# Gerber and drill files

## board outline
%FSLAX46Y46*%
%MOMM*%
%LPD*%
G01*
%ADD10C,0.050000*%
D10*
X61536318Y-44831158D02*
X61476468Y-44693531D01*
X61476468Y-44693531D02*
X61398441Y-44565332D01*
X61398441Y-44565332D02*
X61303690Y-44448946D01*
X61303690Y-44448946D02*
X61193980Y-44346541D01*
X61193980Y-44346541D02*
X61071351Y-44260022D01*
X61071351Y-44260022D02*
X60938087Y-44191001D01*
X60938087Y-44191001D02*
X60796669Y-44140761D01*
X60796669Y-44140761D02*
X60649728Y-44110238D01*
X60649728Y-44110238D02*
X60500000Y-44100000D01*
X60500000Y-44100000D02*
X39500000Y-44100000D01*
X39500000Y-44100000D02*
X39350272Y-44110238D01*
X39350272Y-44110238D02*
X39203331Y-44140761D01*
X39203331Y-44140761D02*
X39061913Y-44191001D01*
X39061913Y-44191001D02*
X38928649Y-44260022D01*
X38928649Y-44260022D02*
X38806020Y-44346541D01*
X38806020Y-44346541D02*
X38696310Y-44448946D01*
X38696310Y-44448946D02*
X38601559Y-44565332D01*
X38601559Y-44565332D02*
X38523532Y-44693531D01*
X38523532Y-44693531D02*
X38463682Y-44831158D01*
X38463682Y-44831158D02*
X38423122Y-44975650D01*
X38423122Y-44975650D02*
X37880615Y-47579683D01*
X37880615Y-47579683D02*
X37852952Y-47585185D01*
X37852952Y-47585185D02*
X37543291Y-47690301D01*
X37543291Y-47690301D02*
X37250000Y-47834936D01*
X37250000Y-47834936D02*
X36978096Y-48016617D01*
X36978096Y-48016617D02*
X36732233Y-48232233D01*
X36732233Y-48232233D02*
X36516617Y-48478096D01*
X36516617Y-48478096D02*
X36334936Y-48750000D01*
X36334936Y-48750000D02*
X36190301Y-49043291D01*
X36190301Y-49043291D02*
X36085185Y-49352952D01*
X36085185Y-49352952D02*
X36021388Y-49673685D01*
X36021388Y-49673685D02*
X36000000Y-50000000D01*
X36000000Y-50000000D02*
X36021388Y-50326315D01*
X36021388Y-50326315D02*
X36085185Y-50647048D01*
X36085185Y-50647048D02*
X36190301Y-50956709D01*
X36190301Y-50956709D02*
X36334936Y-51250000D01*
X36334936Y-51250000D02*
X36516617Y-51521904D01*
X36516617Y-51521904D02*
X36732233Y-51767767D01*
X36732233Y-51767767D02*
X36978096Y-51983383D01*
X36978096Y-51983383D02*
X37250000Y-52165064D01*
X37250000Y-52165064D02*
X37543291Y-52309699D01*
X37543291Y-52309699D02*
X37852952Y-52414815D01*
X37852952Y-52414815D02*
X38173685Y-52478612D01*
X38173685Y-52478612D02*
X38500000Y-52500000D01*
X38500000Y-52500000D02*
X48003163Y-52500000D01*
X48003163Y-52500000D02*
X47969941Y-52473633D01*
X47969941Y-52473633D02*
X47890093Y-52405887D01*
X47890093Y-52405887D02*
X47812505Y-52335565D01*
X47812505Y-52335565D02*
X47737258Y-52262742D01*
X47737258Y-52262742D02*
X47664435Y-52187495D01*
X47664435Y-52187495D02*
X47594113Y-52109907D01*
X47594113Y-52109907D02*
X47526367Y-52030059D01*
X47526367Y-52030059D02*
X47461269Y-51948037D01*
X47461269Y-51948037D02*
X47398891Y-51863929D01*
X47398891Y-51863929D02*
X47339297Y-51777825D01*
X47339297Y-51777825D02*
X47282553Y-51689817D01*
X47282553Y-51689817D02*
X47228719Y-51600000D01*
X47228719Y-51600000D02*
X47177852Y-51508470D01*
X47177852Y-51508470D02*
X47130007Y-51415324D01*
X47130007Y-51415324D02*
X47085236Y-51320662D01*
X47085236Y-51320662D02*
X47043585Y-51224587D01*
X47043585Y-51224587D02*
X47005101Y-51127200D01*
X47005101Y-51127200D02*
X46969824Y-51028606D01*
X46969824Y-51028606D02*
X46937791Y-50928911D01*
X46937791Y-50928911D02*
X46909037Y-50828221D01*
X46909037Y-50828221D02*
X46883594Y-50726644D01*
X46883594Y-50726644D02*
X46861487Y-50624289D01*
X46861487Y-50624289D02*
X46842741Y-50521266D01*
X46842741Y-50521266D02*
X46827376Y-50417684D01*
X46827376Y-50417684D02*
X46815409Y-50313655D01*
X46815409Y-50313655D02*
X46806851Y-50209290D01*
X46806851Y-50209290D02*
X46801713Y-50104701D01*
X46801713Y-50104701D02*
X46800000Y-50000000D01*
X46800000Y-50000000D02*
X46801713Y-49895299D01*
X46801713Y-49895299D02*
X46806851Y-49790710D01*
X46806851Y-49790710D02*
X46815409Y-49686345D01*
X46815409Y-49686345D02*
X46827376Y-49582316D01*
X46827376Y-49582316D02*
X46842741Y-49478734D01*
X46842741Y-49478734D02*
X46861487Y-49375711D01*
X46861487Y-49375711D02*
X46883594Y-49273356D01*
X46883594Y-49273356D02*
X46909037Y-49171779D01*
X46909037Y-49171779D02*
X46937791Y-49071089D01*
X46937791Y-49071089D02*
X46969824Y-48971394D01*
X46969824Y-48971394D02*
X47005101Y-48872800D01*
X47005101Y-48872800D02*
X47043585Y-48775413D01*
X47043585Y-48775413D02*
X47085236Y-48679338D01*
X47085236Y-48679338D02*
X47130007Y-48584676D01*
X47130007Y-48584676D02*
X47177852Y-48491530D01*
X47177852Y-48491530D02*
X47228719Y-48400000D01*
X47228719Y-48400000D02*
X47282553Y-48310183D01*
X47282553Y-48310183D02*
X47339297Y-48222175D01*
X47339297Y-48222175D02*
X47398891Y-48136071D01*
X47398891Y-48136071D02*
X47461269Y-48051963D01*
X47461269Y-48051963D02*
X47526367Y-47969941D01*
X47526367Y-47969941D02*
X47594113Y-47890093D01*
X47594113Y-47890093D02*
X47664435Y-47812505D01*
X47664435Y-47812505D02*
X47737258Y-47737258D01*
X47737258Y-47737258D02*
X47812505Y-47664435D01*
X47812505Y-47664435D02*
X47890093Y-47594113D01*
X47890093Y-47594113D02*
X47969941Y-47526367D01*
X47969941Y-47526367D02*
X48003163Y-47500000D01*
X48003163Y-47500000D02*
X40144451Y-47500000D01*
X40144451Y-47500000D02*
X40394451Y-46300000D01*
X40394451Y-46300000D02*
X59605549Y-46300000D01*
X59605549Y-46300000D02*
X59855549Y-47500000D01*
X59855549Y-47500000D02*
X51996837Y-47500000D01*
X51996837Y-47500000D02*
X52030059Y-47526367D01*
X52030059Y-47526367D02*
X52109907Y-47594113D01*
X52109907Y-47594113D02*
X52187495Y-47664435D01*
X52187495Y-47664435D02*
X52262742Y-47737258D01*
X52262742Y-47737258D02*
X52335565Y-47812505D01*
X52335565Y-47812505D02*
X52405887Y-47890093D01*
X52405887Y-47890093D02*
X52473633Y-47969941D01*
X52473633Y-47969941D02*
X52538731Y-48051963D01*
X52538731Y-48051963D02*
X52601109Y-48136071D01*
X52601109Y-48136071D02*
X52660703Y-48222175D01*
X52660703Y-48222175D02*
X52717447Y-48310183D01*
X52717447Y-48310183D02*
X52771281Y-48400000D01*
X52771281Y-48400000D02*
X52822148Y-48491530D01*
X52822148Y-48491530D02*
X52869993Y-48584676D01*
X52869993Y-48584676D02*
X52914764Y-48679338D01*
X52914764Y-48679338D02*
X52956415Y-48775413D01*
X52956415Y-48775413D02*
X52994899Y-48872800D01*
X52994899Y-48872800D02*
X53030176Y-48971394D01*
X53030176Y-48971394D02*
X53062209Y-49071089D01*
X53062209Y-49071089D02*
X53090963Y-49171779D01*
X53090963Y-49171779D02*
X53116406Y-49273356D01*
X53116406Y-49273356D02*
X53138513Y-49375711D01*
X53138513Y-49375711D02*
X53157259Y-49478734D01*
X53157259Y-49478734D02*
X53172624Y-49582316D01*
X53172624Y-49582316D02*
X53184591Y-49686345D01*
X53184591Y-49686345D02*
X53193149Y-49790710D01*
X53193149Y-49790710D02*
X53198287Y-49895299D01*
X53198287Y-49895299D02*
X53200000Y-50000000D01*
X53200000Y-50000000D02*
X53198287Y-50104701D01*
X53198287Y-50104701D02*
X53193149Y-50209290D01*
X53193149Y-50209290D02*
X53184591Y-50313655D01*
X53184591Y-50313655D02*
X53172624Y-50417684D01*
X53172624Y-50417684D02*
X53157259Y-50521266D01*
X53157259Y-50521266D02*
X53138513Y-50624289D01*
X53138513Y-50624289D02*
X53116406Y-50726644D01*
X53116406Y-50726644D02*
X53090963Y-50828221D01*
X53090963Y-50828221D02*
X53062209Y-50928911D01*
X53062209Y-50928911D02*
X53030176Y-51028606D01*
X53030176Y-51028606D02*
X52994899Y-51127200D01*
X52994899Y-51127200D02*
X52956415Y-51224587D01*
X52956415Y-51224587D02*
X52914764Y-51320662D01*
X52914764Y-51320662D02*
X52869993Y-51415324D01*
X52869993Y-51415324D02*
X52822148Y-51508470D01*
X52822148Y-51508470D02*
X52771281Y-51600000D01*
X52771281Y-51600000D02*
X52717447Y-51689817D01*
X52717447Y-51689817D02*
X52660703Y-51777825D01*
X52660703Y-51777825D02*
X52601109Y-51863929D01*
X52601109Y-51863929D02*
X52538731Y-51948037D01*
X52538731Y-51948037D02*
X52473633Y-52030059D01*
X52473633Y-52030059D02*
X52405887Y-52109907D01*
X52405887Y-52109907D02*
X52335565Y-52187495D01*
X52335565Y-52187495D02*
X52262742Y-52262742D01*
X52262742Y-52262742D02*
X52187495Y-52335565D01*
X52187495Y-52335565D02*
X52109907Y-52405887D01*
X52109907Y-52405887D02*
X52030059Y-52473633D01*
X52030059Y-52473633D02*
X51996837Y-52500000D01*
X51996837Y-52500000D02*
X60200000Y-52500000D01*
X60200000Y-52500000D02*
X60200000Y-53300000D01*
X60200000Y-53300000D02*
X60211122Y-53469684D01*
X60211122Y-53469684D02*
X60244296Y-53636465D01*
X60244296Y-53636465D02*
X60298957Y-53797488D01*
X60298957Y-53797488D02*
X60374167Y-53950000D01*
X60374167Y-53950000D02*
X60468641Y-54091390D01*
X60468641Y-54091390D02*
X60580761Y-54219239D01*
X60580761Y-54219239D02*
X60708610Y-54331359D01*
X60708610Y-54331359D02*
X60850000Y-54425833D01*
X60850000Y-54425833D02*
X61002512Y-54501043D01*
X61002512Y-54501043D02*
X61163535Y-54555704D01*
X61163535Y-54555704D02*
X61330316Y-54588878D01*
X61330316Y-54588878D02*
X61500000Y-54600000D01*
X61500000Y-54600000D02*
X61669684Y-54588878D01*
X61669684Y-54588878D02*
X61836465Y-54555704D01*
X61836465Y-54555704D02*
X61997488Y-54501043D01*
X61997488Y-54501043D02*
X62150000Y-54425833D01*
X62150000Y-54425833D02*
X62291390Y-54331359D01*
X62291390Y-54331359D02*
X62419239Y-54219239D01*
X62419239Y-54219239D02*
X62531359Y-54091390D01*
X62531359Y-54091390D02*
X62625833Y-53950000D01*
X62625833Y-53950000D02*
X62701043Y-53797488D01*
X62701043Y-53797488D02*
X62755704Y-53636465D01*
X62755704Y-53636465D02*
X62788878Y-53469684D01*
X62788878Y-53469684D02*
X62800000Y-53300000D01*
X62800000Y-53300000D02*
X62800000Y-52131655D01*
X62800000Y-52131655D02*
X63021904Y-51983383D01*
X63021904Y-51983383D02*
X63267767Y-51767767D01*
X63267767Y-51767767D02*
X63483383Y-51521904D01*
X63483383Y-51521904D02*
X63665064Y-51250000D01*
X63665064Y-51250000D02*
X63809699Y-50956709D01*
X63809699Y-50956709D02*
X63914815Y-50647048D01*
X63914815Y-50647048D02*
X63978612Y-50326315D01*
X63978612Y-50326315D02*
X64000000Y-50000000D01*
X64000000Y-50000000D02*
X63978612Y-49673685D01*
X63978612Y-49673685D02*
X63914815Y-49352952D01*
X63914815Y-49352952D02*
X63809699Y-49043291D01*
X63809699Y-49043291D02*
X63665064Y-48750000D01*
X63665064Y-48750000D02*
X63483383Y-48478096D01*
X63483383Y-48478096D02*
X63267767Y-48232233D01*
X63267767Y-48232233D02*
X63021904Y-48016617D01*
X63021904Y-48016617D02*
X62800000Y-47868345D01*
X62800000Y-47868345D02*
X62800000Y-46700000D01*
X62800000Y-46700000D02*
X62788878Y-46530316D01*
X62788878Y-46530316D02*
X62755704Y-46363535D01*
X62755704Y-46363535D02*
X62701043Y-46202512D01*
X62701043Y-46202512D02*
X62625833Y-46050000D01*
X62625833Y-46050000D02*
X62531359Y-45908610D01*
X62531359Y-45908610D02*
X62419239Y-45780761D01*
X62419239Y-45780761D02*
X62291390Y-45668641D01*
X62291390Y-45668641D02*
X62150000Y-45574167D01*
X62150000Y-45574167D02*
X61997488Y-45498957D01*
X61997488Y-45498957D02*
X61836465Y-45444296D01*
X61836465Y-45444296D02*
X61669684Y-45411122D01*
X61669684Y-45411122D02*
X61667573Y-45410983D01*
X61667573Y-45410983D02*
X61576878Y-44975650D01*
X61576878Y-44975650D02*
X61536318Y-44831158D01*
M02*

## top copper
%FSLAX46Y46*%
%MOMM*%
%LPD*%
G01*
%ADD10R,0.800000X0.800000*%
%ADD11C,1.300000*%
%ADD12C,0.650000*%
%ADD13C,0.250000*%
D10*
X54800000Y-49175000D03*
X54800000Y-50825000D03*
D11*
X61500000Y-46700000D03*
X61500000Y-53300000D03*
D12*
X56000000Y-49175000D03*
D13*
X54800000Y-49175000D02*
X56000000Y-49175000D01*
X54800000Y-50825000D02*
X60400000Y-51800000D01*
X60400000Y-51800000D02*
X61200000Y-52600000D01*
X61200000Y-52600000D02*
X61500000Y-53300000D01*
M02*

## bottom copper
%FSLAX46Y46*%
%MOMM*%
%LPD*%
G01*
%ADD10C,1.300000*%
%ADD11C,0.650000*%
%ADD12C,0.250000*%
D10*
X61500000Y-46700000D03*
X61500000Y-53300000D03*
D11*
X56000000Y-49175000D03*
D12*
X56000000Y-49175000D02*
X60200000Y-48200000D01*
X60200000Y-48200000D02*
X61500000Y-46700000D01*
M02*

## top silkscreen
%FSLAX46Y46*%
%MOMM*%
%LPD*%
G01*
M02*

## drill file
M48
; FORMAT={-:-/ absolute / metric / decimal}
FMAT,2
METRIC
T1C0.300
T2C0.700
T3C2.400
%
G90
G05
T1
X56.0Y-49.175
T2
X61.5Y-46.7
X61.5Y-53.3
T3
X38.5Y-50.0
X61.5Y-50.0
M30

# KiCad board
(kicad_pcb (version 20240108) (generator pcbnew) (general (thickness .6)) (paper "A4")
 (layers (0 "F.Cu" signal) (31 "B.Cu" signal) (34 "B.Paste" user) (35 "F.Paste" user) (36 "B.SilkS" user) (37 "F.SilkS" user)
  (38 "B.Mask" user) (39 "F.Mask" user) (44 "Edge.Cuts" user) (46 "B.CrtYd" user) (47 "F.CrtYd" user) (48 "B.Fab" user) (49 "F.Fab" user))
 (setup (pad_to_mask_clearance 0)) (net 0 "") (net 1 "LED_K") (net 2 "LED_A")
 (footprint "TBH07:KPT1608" (layer "F.Cu") (at 54.8 50)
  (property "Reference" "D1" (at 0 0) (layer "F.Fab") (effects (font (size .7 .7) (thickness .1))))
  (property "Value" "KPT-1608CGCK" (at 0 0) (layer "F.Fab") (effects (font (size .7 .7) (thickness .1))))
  (pad "1" smd rect (at 0 -.825) (size .8 .8) (layers "F.Cu" "F.Paste" "F.Mask") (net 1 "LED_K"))
  (pad "2" smd rect (at 0 .825) (size .8 .8) (layers "F.Cu" "F.Paste" "F.Mask") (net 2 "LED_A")))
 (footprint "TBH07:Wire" (layer "F.Cu") (at 61.5 46.7)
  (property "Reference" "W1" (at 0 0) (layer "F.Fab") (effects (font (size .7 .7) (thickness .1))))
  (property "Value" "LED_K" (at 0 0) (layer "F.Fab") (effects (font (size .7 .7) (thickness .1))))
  (pad "1" thru_hole circle (at 0 0) (size 1.3 1.3) (drill .7) (layers "*.Cu" "*.Mask") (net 1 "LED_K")))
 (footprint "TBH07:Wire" (layer "F.Cu") (at 61.5 53.3)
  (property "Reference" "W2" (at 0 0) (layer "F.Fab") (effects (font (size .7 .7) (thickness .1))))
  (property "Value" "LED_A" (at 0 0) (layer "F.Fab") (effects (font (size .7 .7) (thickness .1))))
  (pad "1" thru_hole circle (at 0 0) (size 1.3 1.3) (drill .7) (layers "*.Cu" "*.Mask") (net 2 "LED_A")))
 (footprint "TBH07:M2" (layer "F.Cu") (at 38.5 50)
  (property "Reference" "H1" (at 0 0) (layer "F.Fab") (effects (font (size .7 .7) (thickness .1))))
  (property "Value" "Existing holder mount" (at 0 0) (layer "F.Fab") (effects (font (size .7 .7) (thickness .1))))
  (pad "" np_thru_hole circle (at 0 0) (size 2.4 2.4) (drill 2.4) (layers "*.Cu" "*.Mask")))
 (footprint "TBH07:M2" (layer "F.Cu") (at 61.5 50)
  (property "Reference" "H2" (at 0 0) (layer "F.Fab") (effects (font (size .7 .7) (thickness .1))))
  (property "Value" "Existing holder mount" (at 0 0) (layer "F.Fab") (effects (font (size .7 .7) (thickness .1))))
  (pad "" np_thru_hole circle (at 0 0) (size 2.4 2.4) (drill 2.4) (layers "*.Cu" "*.Mask")))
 (segment (start 54.8 49.175) (end 56 49.175) (width .25) (layer "F.Cu") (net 1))
 (via (at 56 49.175) (size .65) (drill .3) (layers "F.Cu" "B.Cu") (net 1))
 (segment (start 56 49.175) (end 60.2 48.2) (width .25) (layer "B.Cu") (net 1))
 (segment (start 60.2 48.2) (end 61.5 46.7) (width .25) (layer "B.Cu") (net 1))
 (segment (start 54.8 50.825) (end 60.4 51.8) (width .25) (layer "F.Cu") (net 2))
 (segment (start 60.4 51.8) (end 61.2 52.6) (width .25) (layer "F.Cu") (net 2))
 (segment (start 61.2 52.6) (end 61.5 53.3) (width .25) (layer "F.Cu") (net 2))
 (gr_line (start 61.5363181856797 44.831157732859225) (end 61.47646762268844 44.69353086782984) (stroke (width .05) (type default))
  (layer "Edge.Cuts"))
 (gr_line (start 61.47646762268844 44.69353086782984) (end 61.39844084614742 44.56533154641664) (stroke (width .05) (type default))
  (layer "Edge.Cuts"))
 (gr_line (start 61.39844084614742 44.56533154641664) (end 61.30369026607012 44.448946102983186) (stroke (width .05) (type default))
  (layer "Edge.Cuts"))
 (gr_line (start 61.30369026607012 44.448946102983186) (end 61.19397959354886 44.34654096540152) (stroke (width .05) (type default))
  (layer "Edge.Cuts"))
 (gr_line (start 61.19397959354886 44.34654096540152) (end 61.07135101059367 44.26002232861967) (stroke (width .05) (type default))
  (layer "Edge.Cuts"))
 (gr_line (start 61.07135101059367 44.26002232861967) (end 60.9380871564435 44.19100067227017) (stroke (width .05) (type default))
  (layer "Edge.Cuts"))
 (gr_line (start 60.9380871564435 44.19100067227017) (end 60.79666863794614 44.14076078279778) (stroke (width .05) (type default))
  (layer "Edge.Cuts"))
 (gr_line (start 60.79666863794614 44.14076078279778) (end 60.64972785491944 44.110237838121904) (stroke (width .05) (type default))
  (layer "Edge.Cuts"))
 (gr_line (start 60.64972785491944 44.110237838121904) (end 60.5 44.1) (stroke (width .05) (type default)) (layer "Edge.Cuts"))
 (gr_line (start 60.5 44.1) (end 39.5 44.1) (stroke (width .05) (type default)) (layer "Edge.Cuts"))
 (gr_line (start 39.5 44.1) (end 39.35027214508056 44.110237838121904) (stroke (width .05) (type default)) (layer "Edge.Cuts"))
 (gr_line (start 39.35027214508056 44.110237838121904) (end 39.20333136205386 44.14076078279778) (stroke (width .05) (type default))
  (layer "Edge.Cuts"))
 (gr_line (start 39.20333136205386 44.14076078279778) (end 39.0619128435565 44.19100067227017) (stroke (width .05) (type default))
  (layer "Edge.Cuts"))
 (gr_line (start 39.0619128435565 44.19100067227017) (end 38.92864898940633 44.26002232861967) (stroke (width .05) (type default))
  (layer "Edge.Cuts"))
 (gr_line (start 38.92864898940633 44.26002232861967) (end 38.80602040645114 44.34654096540152) (stroke (width .05) (type default))
  (layer "Edge.Cuts"))
 (gr_line (start 38.80602040645114 44.34654096540152) (end 38.69630973392988 44.448946102983186) (stroke (width .05) (type default))
  (layer "Edge.Cuts"))
 (gr_line (start 38.69630973392988 44.448946102983186) (end 38.60155915385258 44.56533154641664) (stroke (width .05) (type default))
  (layer "Edge.Cuts"))
 (gr_line (start 38.60155915385258 44.56533154641664) (end 38.52353237731156 44.69353086782984) (stroke (width .05) (type default))
  (layer "Edge.Cuts"))
 (gr_line (start 38.52353237731156 44.69353086782984) (end 38.4636818143203 44.831157732859225) (stroke (width .05) (type default))
  (layer "Edge.Cuts"))
 (gr_line (start 38.4636818143203 44.831157732859225) (end 38.42312153828863 44.9756503204768) (stroke (width .05) (type default))
  (layer "Edge.Cuts"))
 (gr_line (start 38.42312153828863 44.9756503204768) (end 37.8806147187135 47.57968305443743) (stroke (width .05) (type default))
  (layer "Edge.Cuts"))
 (gr_line (start 37.8806147187135 47.57968305443743) (end 37.8529523872437 47.58518543427733) (stroke (width .05) (type default))
  (layer "Edge.Cuts"))
 (gr_line (start 37.8529523872437 47.58518543427733) (end 37.543291419087275 47.69030116872178) (stroke (width .05) (type default))
  (layer "Edge.Cuts"))
 (gr_line (start 37.543291419087275 47.69030116872178) (end 37.25 47.8349364905389) (stroke (width .05) (type default)) (layer "Edge.Cuts"))
 (gr_line (start 37.25 47.8349364905389) (end 36.9780964274782 48.01661664927191) (stroke (width .05) (type default)) (layer "Edge.Cuts"))
 (gr_line (start 36.9780964274782 48.01661664927191) (end 36.73223304703363 48.23223304703363) (stroke (width .05) (type default))
  (layer "Edge.Cuts"))
 (gr_line (start 36.73223304703363 48.23223304703363) (end 36.51661664927191 48.4780964274782) (stroke (width .05) (type default))
  (layer "Edge.Cuts"))
 (gr_line (start 36.51661664927191 48.4780964274782) (end 36.33493649053891 48.75) (stroke (width .05) (type default)) (layer "Edge.Cuts"))
 (gr_line (start 36.33493649053891 48.75) (end 36.19030116872178 49.043291419087275) (stroke (width .05) (type default)) (layer "Edge.Cuts"))
 (gr_line (start 36.19030116872178 49.043291419087275) (end 36.08518543427733 49.3529523872437) (stroke (width .05) (type default))
  (layer "Edge.Cuts"))
 (gr_line (start 36.08518543427733 49.3529523872437) (end 36.021387846565474 49.67368451944987) (stroke (width .05) (type default))
  (layer "Edge.Cuts"))
 (gr_line (start 36.021387846565474 49.67368451944987) (end 36.0 50.0) (stroke (width .05) (type default)) (layer "Edge.Cuts"))
 (gr_line (start 36.0 50.0) (end 36.021387846565474 50.32631548055013) (stroke (width .05) (type default)) (layer "Edge.Cuts"))
 (gr_line (start 36.021387846565474 50.32631548055013) (end 36.08518543427733 50.6470476127563) (stroke (width .05) (type default))
  (layer "Edge.Cuts"))
 (gr_line (start 36.08518543427733 50.6470476127563) (end 36.19030116872178 50.956708580912725) (stroke (width .05) (type default))
  (layer "Edge.Cuts"))
 (gr_line (start 36.19030116872178 50.956708580912725) (end 36.3349364905389 51.25) (stroke (width .05) (type default)) (layer "Edge.Cuts"))
 (gr_line (start 36.3349364905389 51.25) (end 36.51661664927191 51.5219035725218) (stroke (width .05) (type default)) (layer "Edge.Cuts"))
 (gr_line (start 36.51661664927191 51.5219035725218) (end 36.73223304703363 51.76776695296637) (stroke (width .05) (type default))
  (layer "Edge.Cuts"))
 (gr_line (start 36.73223304703363 51.76776695296637) (end 36.9780964274782 51.98338335072809) (stroke (width .05) (type default))
  (layer "Edge.Cuts"))
 (gr_line (start 36.9780964274782 51.98338335072809) (end 37.25 52.1650635094611) (stroke (width .05) (type default)) (layer "Edge.Cuts"))
 (gr_line (start 37.25 52.1650635094611) (end 37.543291419087275 52.30969883127822) (stroke (width .05) (type default)) (layer "Edge.Cuts"))
 (gr_line (start 37.543291419087275 52.30969883127822) (end 37.8529523872437 52.41481456572267) (stroke (width .05) (type default))
  (layer "Edge.Cuts"))
 (gr_line (start 37.8529523872437 52.41481456572267) (end 38.17368451944987 52.478612153434526) (stroke (width .05) (type default))
  (layer "Edge.Cuts"))
 (gr_line (start 38.17368451944987 52.478612153434526) (end 38.5 52.5) (stroke (width .05) (type default)) (layer "Edge.Cuts"))
 (gr_line (start 38.5 52.5) (end 48.00316310634037 52.5) (stroke (width .05) (type default)) (layer "Edge.Cuts"))
 (gr_line (start 48.00316310634037 52.5) (end 47.969941490676334 52.47363345076076) (stroke (width .05) (type default)) (layer "Edge.Cuts"))
 (gr_line (start 47.969941490676334 52.47363345076076) (end 47.89009339167978 52.40588738393273) (stroke (width .05) (type default))
  (layer "Edge.Cuts"))
 (gr_line (start 47.89009339167978 52.40588738393273) (end 47.812504633526814 52.33556503263307) (stroke (width .05) (type default))
  (layer "Edge.Cuts"))
 (gr_line (start 47.812504633526814 52.33556503263307) (end 47.737258300203045 52.26274169979695) (stroke (width .05) (type default))
  (layer "Edge.Cuts"))
 (gr_line (start 47.737258300203045 52.26274169979695) (end 47.66443496736692 52.187495366473186) (stroke (width .05) (type default))
  (layer "Edge.Cuts"))
 (gr_line (start 47.66443496736692 52.187495366473186) (end 47.59411261606727 52.109906608320216) (stroke (width .05) (type default))
  (layer "Edge.Cuts"))
 (gr_line (start 47.59411261606727 52.109906608320216) (end 47.52636654923924 52.030058509323666) (stroke (width .05) (type default))
  (layer "Edge.Cuts"))
 (gr_line (start 47.52636654923924 52.030058509323666) (end 47.461269311068044 51.9480365728279) (stroke (width .05) (type default))
  (layer "Edge.Cuts"))
 (gr_line (start 47.461269311068044 51.9480365728279) (end 47.39889060930683 51.86392862997697) (stroke (width .05) (type default))
  (layer "Edge.Cuts"))
 (gr_line (start 47.39889060930683 51.86392862997697) (end 47.33929724063185 51.77782474566273) (stroke (width .05) (type default))
  (layer "Edge.Cuts"))
 (gr_line (start 47.33929724063185 51.77782474566273) (end 47.28255301911494 51.68981712208117) (stroke (width .05) (type default))
  (layer "Edge.Cuts"))
 (gr_line (start 47.28255301911494 51.68981712208117) (end 47.2287187078898 51.6) (stroke (width .05) (type default)) (layer "Edge.Cuts"))
 (gr_line (start 47.2287187078898 51.6) (end 47.17785195408526 51.50846955784319) (stroke (width .05) (type default)) (layer "Edge.Cuts"))
 (gr_line (start 47.17785195408526 51.50846955784319) (end 47.1300072270954 51.415323808700805) (stroke (width .05) (type default))
  (layer "Edge.Cuts"))
 (gr_line (start 47.1300072270954 51.415323808700805) (end 47.08523576025224 51.320662495374066) (stroke (width .05) (type default))
  (layer "Edge.Cuts"))
 (gr_line (start 47.08523576025224 51.320662495374066) (end 47.04358549596388 51.22458698356829) (stroke (width .05) (type default))
  (layer "Edge.Cuts"))
 (gr_line (start 47.04358549596388 51.22458698356829) (end 47.00510103437656 51.12720015334795) (stroke (width .05) (type default))
  (layer "Edge.Cuts"))
 (gr_line (start 47.00510103437656 51.12720015334795) (end 46.969823585615664 51.02860628897012) (stroke (width .05) (type default))
  (layer "Edge.Cuts"))
 (gr_line (start 46.969823585615664 51.02860628897012) (end 46.937790925656934 50.92891096721428) (stroke (width .05) (type default))
  (layer "Edge.Cuts"))
 (gr_line (start 46.937790925656934 50.92891096721428) (end 46.90903735587498 50.828220944328066) (stroke (width .05) (type default))
  (layer "Edge.Cuts"))
 (gr_line (start 46.90903735587498 50.828220944328066) (end 46.883593666312535 50.726644041709996) (stroke (width .05) (type default))
  (layer "Edge.Cuts"))
 (gr_line (start 46.883593666312535 50.726644041709996) (end 46.86148710270966 50.62428903045161) (stroke (width .05) (type default))
  (layer "Edge.Cuts"))
 (gr_line (start 46.86148710270966 50.62428903045161) (end 46.842741337328384 50.521265514862684) (stroke (width .05) (type default))
  (layer "Edge.Cuts"))
 (gr_line (start 46.842741337328384 50.521265514862684) (end 46.827376443603804 50.41768381510416) (stroke (width .05) (type default))
  (layer "Edge.Cuts"))
 (gr_line (start 46.827376443603804 50.41768381510416) (end 46.815408874648966 50.31365484905459) (stroke (width .05) (type default))
  (layer "Edge.Cuts"))
 (gr_line (start 46.815408874648966 50.31365484905459) (end 46.80685144563647 50.20929001353646) (stroke (width .05) (type default))
  (layer "Edge.Cuts"))
 (gr_line (start 46.80685144563647 50.20929001353646) (end 46.80171332007563 50.10470106502968) (stroke (width .05) (type default))
  (layer "Edge.Cuts"))
 (gr_line (start 46.80171332007563 50.10470106502968) (end 46.8 50.0) (stroke (width .05) (type default)) (layer "Edge.Cuts"))
 (gr_line (start 46.8 50.0) (end 46.80171332007563 49.89529893497031) (stroke (width .05) (type default)) (layer "Edge.Cuts"))
 (gr_line (start 46.80171332007563 49.89529893497031) (end 46.80685144563647 49.79070998646354) (stroke (width .05) (type default))
  (layer "Edge.Cuts"))
 (gr_line (start 46.80685144563647 49.79070998646354) (end 46.815408874648966 49.68634515094541) (stroke (width .05) (type default))
  (layer "Edge.Cuts"))
 (gr_line (start 46.815408874648966 49.68634515094541) (end 46.827376443603804 49.58231618489583) (stroke (width .05) (type default))
  (layer "Edge.Cuts"))
 (gr_line (start 46.827376443603804 49.58231618489583) (end 46.842741337328384 49.478734485137316) (stroke (width .05) (type default))
  (layer "Edge.Cuts"))
 (gr_line (start 46.842741337328384 49.478734485137316) (end 46.86148710270966 49.375710969548386) (stroke (width .05) (type default))
  (layer "Edge.Cuts"))
 (gr_line (start 46.86148710270966 49.375710969548386) (end 46.883593666312535 49.273355958290004) (stroke (width .05) (type default))
  (layer "Edge.Cuts"))
 (gr_line (start 46.883593666312535 49.273355958290004) (end 46.90903735587498 49.171779055671934) (stroke (width .05) (type default))
  (layer "Edge.Cuts"))
 (gr_line (start 46.90903735587498 49.171779055671934) (end 46.937790925656934 49.07108903278572) (stroke (width .05) (type default))
  (layer "Edge.Cuts"))
 (gr_line (start 46.937790925656934 49.07108903278572) (end 46.969823585615664 48.97139371102988) (stroke (width .05) (type default))
  (layer "Edge.Cuts"))
 (gr_line (start 46.969823585615664 48.97139371102988) (end 47.00510103437656 48.87279984665205) (stroke (width .05) (type default))
  (layer "Edge.Cuts"))
 (gr_line (start 47.00510103437656 48.87279984665205) (end 47.04358549596388 48.77541301643171) (stroke (width .05) (type default))
  (layer "Edge.Cuts"))
 (gr_line (start 47.04358549596388 48.77541301643171) (end 47.08523576025224 48.679337504625934) (stroke (width .05) (type default))
  (layer "Edge.Cuts"))
 (gr_line (start 47.08523576025224 48.679337504625934) (end 47.1300072270954 48.584676191299195) (stroke (width .05) (type default))
  (layer "Edge.Cuts"))
 (gr_line (start 47.1300072270954 48.584676191299195) (end 47.17785195408526 48.49153044215681) (stroke (width .05) (type default))
  (layer "Edge.Cuts"))
 (gr_line (start 47.17785195408526 48.49153044215681) (end 47.2287187078898 48.4) (stroke (width .05) (type default)) (layer "Edge.Cuts"))
 (gr_line (start 47.2287187078898 48.4) (end 47.28255301911495 48.31018287791882) (stroke (width .05) (type default)) (layer "Edge.Cuts"))
 (gr_line (start 47.28255301911495 48.31018287791882) (end 47.33929724063186 48.22217525433727) (stroke (width .05) (type default))
  (layer "Edge.Cuts"))
 (gr_line (start 47.33929724063186 48.22217525433727) (end 47.39889060930683 48.13607137002303) (stroke (width .05) (type default))
  (layer "Edge.Cuts"))
 (gr_line (start 47.39889060930683 48.13607137002303) (end 47.46126931106805 48.05196342717209) (stroke (width .05) (type default))
  (layer "Edge.Cuts"))
 (gr_line (start 47.46126931106805 48.05196342717209) (end 47.52636654923924 47.969941490676334) (stroke (width .05) (type default))
  (layer "Edge.Cuts"))
 (gr_line (start 47.52636654923924 47.969941490676334) (end 47.59411261606727 47.89009339167978) (stroke (width .05) (type default))
  (layer "Edge.Cuts"))
 (gr_line (start 47.59411261606727 47.89009339167978) (end 47.66443496736693 47.812504633526814) (stroke (width .05) (type default))
  (layer "Edge.Cuts"))
 (gr_line (start 47.66443496736693 47.812504633526814) (end 47.737258300203045 47.737258300203045) (stroke (width .05) (type default))
  (layer "Edge.Cuts"))
 (gr_line (start 47.737258300203045 47.737258300203045) (end 47.812504633526814 47.66443496736692) (stroke (width .05) (type default))
  (layer "Edge.Cuts"))
 (gr_line (start 47.812504633526814 47.66443496736692) (end 47.890093391679784 47.59411261606727) (stroke (width .05) (type default))
  (layer "Edge.Cuts"))
 (gr_line (start 47.890093391679784 47.59411261606727) (end 47.969941490676334 47.52636654923924) (stroke (width .05) (type default))
  (layer "Edge.Cuts"))
 (gr_line (start 47.969941490676334 47.52636654923924) (end 48.00316310634037 47.5) (stroke (width .05) (type default)) (layer "Edge.Cuts"))
 (gr_line (start 48.00316310634037 47.5) (end 40.14445131161203 47.5) (stroke (width .05) (type default)) (layer "Edge.Cuts"))
 (gr_line (start 40.14445131161203 47.5) (end 40.39445131161203 46.3) (stroke (width .05) (type default)) (layer "Edge.Cuts"))
 (gr_line (start 40.39445131161203 46.3) (end 59.60554868838797 46.3) (stroke (width .05) (type default)) (layer "Edge.Cuts"))
 (gr_line (start 59.60554868838797 46.3) (end 59.85554868838797 47.5) (stroke (width .05) (type default)) (layer "Edge.Cuts"))
 (gr_line (start 59.85554868838797 47.5) (end 51.99683689365963 47.5) (stroke (width .05) (type default)) (layer "Edge.Cuts"))
 (gr_line (start 51.99683689365963 47.5) (end 52.030058509323666 47.52636654923924) (stroke (width .05) (type default)) (layer "Edge.Cuts"))
 (gr_line (start 52.030058509323666 47.52636654923924) (end 52.10990660832022 47.59411261606727) (stroke (width .05) (type default))
  (layer "Edge.Cuts"))
 (gr_line (start 52.10990660832022 47.59411261606727) (end 52.187495366473186 47.66443496736693) (stroke (width .05) (type default))
  (layer "Edge.Cuts"))
 (gr_line (start 52.187495366473186 47.66443496736693) (end 52.262741699796955 47.737258300203045) (stroke (width .05) (type default))
  (layer "Edge.Cuts"))
 (gr_line (start 52.262741699796955 47.737258300203045) (end 52.33556503263308 47.812504633526814) (stroke (width .05) (type default))
  (layer "Edge.Cuts"))
 (gr_line (start 52.33556503263308 47.812504633526814) (end 52.40588738393273 47.89009339167978) (stroke (width .05) (type default))
  (layer "Edge.Cuts"))
 (gr_line (start 52.40588738393273 47.89009339167978) (end 52.47363345076076 47.969941490676334) (stroke (width .05) (type default))
  (layer "Edge.Cuts"))
 (gr_line (start 52.47363345076076 47.969941490676334) (end 52.538730688931956 48.0519634271721) (stroke (width .05) (type default))
  (layer "Edge.Cuts"))
 (gr_line (start 52.538730688931956 48.0519634271721) (end 52.60110939069317 48.13607137002303) (stroke (width .05) (type default))
  (layer "Edge.Cuts"))
 (gr_line (start 52.60110939069317 48.13607137002303) (end 52.66070275936814 48.22217525433727) (stroke (width .05) (type default))
  (layer "Edge.Cuts"))
 (gr_line (start 52.66070275936814 48.22217525433727) (end 52.71744698088505 48.31018287791882) (stroke (width .05) (type default))
  (layer "Edge.Cuts"))
 (gr_line (start 52.71744698088505 48.31018287791882) (end 52.7712812921102 48.4) (stroke (width .05) (type default)) (layer "Edge.Cuts"))
 (gr_line (start 52.7712812921102 48.4) (end 52.82214804591474 48.49153044215681) (stroke (width .05) (type default)) (layer "Edge.Cuts"))
 (gr_line (start 52.82214804591474 48.49153044215681) (end 52.8699927729046 48.584676191299195) (stroke (width .05) (type default))
  (layer "Edge.Cuts"))
 (gr_line (start 52.8699927729046 48.584676191299195) (end 52.91476423974776 48.679337504625934) (stroke (width .05) (type default))
  (layer "Edge.Cuts"))
 (gr_line (start 52.91476423974776 48.679337504625934) (end 52.95641450403612 48.77541301643171) (stroke (width .05) (type default))
  (layer "Edge.Cuts"))
 (gr_line (start 52.95641450403612 48.77541301643171) (end 52.99489896562344 48.87279984665205) (stroke (width .05) (type default))
  (layer "Edge.Cuts"))
 (gr_line (start 52.99489896562344 48.87279984665205) (end 53.030176414384336 48.97139371102988) (stroke (width .05) (type default))
  (layer "Edge.Cuts"))
 (gr_line (start 53.030176414384336 48.97139371102988) (end 53.062209074343066 49.07108903278572) (stroke (width .05) (type default))
  (layer "Edge.Cuts"))
 (gr_line (start 53.062209074343066 49.07108903278572) (end 53.09096264412502 49.171779055671934) (stroke (width .05) (type default))
  (layer "Edge.Cuts"))
 (gr_line (start 53.09096264412502 49.171779055671934) (end 53.116406333687465 49.273355958290004) (stroke (width .05) (type default))
  (layer "Edge.Cuts"))
 (gr_line (start 53.116406333687465 49.273355958290004) (end 53.13851289729034 49.375710969548386) (stroke (width .05) (type default))
  (layer "Edge.Cuts"))
 (gr_line (start 53.13851289729034 49.375710969548386) (end 53.157258662671616 49.478734485137316) (stroke (width .05) (type default))
  (layer "Edge.Cuts"))
 (gr_line (start 53.157258662671616 49.478734485137316) (end 53.172623556396196 49.58231618489584) (stroke (width .05) (type default))
  (layer "Edge.Cuts"))
 (gr_line (start 53.172623556396196 49.58231618489584) (end 53.184591125351034 49.68634515094541) (stroke (width .05) (type default))
  (layer "Edge.Cuts"))
 (gr_line (start 53.184591125351034 49.68634515094541) (end 53.19314855436353 49.79070998646354) (stroke (width .05) (type default))
  (layer "Edge.Cuts"))
 (gr_line (start 53.19314855436353 49.79070998646354) (end 53.19828667992437 49.89529893497031) (stroke (width .05) (type default))
  (layer "Edge.Cuts"))
 (gr_line (start 53.19828667992437 49.89529893497031) (end 53.2 50.0) (stroke (width .05) (type default)) (layer "Edge.Cuts"))
 (gr_line (start 53.2 50.0) (end 53.19828667992437 50.10470106502969) (stroke (width .05) (type default)) (layer "Edge.Cuts"))
 (gr_line (start 53.19828667992437 50.10470106502969) (end 53.19314855436353 50.20929001353646) (stroke (width .05) (type default))
  (layer "Edge.Cuts"))
 (gr_line (start 53.19314855436353 50.20929001353646) (end 53.184591125351034 50.31365484905459) (stroke (width .05) (type default))
  (layer "Edge.Cuts"))
 (gr_line (start 53.184591125351034 50.31365484905459) (end 53.17262355639619 50.41768381510417) (stroke (width .05) (type default))
  (layer "Edge.Cuts"))
 (gr_line (start 53.17262355639619 50.41768381510417) (end 53.157258662671616 50.521265514862684) (stroke (width .05) (type default))
  (layer "Edge.Cuts"))
 (gr_line (start 53.157258662671616 50.521265514862684) (end 53.13851289729034 50.624289030451614) (stroke (width .05) (type default))
  (layer "Edge.Cuts"))
 (gr_line (start 53.13851289729034 50.624289030451614) (end 53.116406333687465 50.726644041709996) (stroke (width .05) (type default))
  (layer "Edge.Cuts"))
 (gr_line (start 53.116406333687465 50.726644041709996) (end 53.09096264412502 50.828220944328066) (stroke (width .05) (type default))
  (layer "Edge.Cuts"))
 (gr_line (start 53.09096264412502 50.828220944328066) (end 53.062209074343066 50.928910967214286) (stroke (width .05) (type default))
  (layer "Edge.Cuts"))
 (gr_line (start 53.062209074343066 50.928910967214286) (end 53.030176414384336 51.02860628897012) (stroke (width .05) (type default))
  (layer "Edge.Cuts"))
 (gr_line (start 53.030176414384336 51.02860628897012) (end 52.99489896562344 51.12720015334795) (stroke (width .05) (type default))
  (layer "Edge.Cuts"))
 (gr_line (start 52.99489896562344 51.12720015334795) (end 52.95641450403612 51.22458698356829) (stroke (width .05) (type default))
  (layer "Edge.Cuts"))
 (gr_line (start 52.95641450403612 51.22458698356829) (end 52.91476423974776 51.320662495374066) (stroke (width .05) (type default))
  (layer "Edge.Cuts"))
 (gr_line (start 52.91476423974776 51.320662495374066) (end 52.8699927729046 51.415323808700805) (stroke (width .05) (type default))
  (layer "Edge.Cuts"))
 (gr_line (start 52.8699927729046 51.415323808700805) (end 52.82214804591474 51.50846955784319) (stroke (width .05) (type default))
  (layer "Edge.Cuts"))
 (gr_line (start 52.82214804591474 51.50846955784319) (end 52.7712812921102 51.6) (stroke (width .05) (type default)) (layer "Edge.Cuts"))
 (gr_line (start 52.7712812921102 51.6) (end 52.71744698088505 51.68981712208118) (stroke (width .05) (type default)) (layer "Edge.Cuts"))
 (gr_line (start 52.71744698088505 51.68981712208118) (end 52.66070275936814 51.77782474566273) (stroke (width .05) (type default))
  (layer "Edge.Cuts"))
 (gr_line (start 52.66070275936814 51.77782474566273) (end 52.60110939069317 51.86392862997697) (stroke (width .05) (type default))
  (layer "Edge.Cuts"))
 (gr_line (start 52.60110939069317 51.86392862997697) (end 52.53873068893195 51.94803657282791) (stroke (width .05) (type default))
  (layer "Edge.Cuts"))
 (gr_line (start 52.53873068893195 51.94803657282791) (end 52.47363345076076 52.030058509323666) (stroke (width .05) (type default))
  (layer "Edge.Cuts"))
 (gr_line (start 52.47363345076076 52.030058509323666) (end 52.40588738393273 52.10990660832022) (stroke (width .05) (type default))
  (layer "Edge.Cuts"))
 (gr_line (start 52.40588738393273 52.10990660832022) (end 52.33556503263307 52.18749536647319) (stroke (width .05) (type default))
  (layer "Edge.Cuts"))
 (gr_line (start 52.33556503263307 52.18749536647319) (end 52.262741699796955 52.262741699796955) (stroke (width .05) (type default))
  (layer "Edge.Cuts"))
 (gr_line (start 52.262741699796955 52.262741699796955) (end 52.187495366473186 52.33556503263308) (stroke (width .05) (type default))
  (layer "Edge.Cuts"))
 (gr_line (start 52.187495366473186 52.33556503263308) (end 52.109906608320216 52.40588738393273) (stroke (width .05) (type default))
  (layer "Edge.Cuts"))
 (gr_line (start 52.109906608320216 52.40588738393273) (end 52.030058509323666 52.47363345076076) (stroke (width .05) (type default))
  (layer "Edge.Cuts"))
 (gr_line (start 52.030058509323666 52.47363345076076) (end 51.99683689365963 52.5) (stroke (width .05) (type default)) (layer "Edge.Cuts"))
 (gr_line (start 51.99683689365963 52.5) (end 60.2 52.5) (stroke (width .05) (type default)) (layer "Edge.Cuts"))
 (gr_line (start 60.2 52.5) (end 60.2 53.3) (stroke (width .05) (type default)) (layer "Edge.Cuts"))
 (gr_line (start 60.2 53.3) (end 60.21112168021405 53.46968404988607) (stroke (width .05) (type default)) (layer "Edge.Cuts"))
 (gr_line (start 60.21112168021405 53.46968404988607) (end 60.24429642582421 53.63646475863328) (stroke (width .05) (type default))
  (layer "Edge.Cuts"))
 (gr_line (start 60.24429642582421 53.63646475863328) (end 60.29895660773533 53.79748846207462) (stroke (width .05) (type default))
  (layer "Edge.Cuts"))
 (gr_line (start 60.29895660773533 53.79748846207462) (end 60.37416697508023 53.95) (stroke (width .05) (type default)) (layer "Edge.Cuts"))
 (gr_line (start 60.37416697508023 53.95) (end 60.46864065762139 54.091389857711334) (stroke (width .05) (type default)) (layer "Edge.Cuts"))
 (gr_line (start 60.46864065762139 54.091389857711334) (end 60.58076118445749 54.21923881554251) (stroke (width .05) (type default))
  (layer "Edge.Cuts"))
 (gr_line (start 60.58076118445749 54.21923881554251) (end 60.70861014228866 54.331359342378605) (stroke (width .05) (type default))
  (layer "Edge.Cuts"))
 (gr_line (start 60.70861014228866 54.331359342378605) (end 60.85 54.42583302491977) (stroke (width .05) (type default)) (layer "Edge.Cuts"))
 (gr_line (start 60.85 54.42583302491977) (end 61.002511537925386 54.50104339226467) (stroke (width .05) (type default)) (layer "Edge.Cuts"))
 (gr_line (start 61.002511537925386 54.50104339226467) (end 61.16353524136672 54.55570357417579) (stroke (width .05) (type default))
  (layer "Edge.Cuts"))
 (gr_line (start 61.16353524136672 54.55570357417579) (end 61.330315950113935 54.588878319785955) (stroke (width .05) (type default))
  (layer "Edge.Cuts"))
 (gr_line (start 61.330315950113935 54.588878319785955) (end 61.5 54.6) (stroke (width .05) (type default)) (layer "Edge.Cuts"))
 (gr_line (start 61.5 54.6) (end 61.669684049886065 54.588878319785955) (stroke (width .05) (type default)) (layer "Edge.Cuts"))
 (gr_line (start 61.669684049886065 54.588878319785955) (end 61.83646475863328 54.55570357417579) (stroke (width .05) (type default))
  (layer "Edge.Cuts"))
 (gr_line (start 61.83646475863328 54.55570357417579) (end 61.997488462074614 54.50104339226468) (stroke (width .05) (type default))
  (layer "Edge.Cuts"))
 (gr_line (start 61.997488462074614 54.50104339226468) (end 62.15 54.42583302491977) (stroke (width .05) (type default)) (layer "Edge.Cuts"))
 (gr_line (start 62.15 54.42583302491977) (end 62.29138985771134 54.331359342378605) (stroke (width .05) (type default)) (layer "Edge.Cuts"))
 (gr_line (start 62.29138985771134 54.331359342378605) (end 62.41923881554251 54.21923881554251) (stroke (width .05) (type default))
  (layer "Edge.Cuts"))
 (gr_line (start 62.41923881554251 54.21923881554251) (end 62.53135934237861 54.091389857711334) (stroke (width .05) (type default))
  (layer "Edge.Cuts"))
 (gr_line (start 62.53135934237861 54.091389857711334) (end 62.62583302491977 53.95) (stroke (width .05) (type default)) (layer "Edge.Cuts"))
 (gr_line (start 62.62583302491977 53.95) (end 62.70104339226467 53.79748846207462) (stroke (width .05) (type default)) (layer "Edge.Cuts"))
 (gr_line (start 62.70104339226467 53.79748846207462) (end 62.75570357417579 53.63646475863328) (stroke (width .05) (type default))
  (layer "Edge.Cuts"))
 (gr_line (start 62.75570357417579 53.63646475863328) (end 62.78887831978595 53.46968404988607) (stroke (width .05) (type default))
  (layer "Edge.Cuts"))
 (gr_line (start 62.78887831978595 53.46968404988607) (end 62.8 53.3) (stroke (width .05) (type default)) (layer "Edge.Cuts"))
 (gr_line (start 62.8 53.3) (end 62.8 52.13165457756513) (stroke (width .05) (type default)) (layer "Edge.Cuts"))
 (gr_line (start 62.8 52.13165457756513) (end 63.0219035725218 51.98338335072809) (stroke (width .05) (type default)) (layer "Edge.Cuts"))
 (gr_line (start 63.0219035725218 51.98338335072809) (end 63.26776695296637 51.76776695296637) (stroke (width .05) (type default))
  (layer "Edge.Cuts"))
 (gr_line (start 63.26776695296637 51.76776695296637) (end 63.48338335072809 51.5219035725218) (stroke (width .05) (type default))
  (layer "Edge.Cuts"))
 (gr_line (start 63.48338335072809 51.5219035725218) (end 63.66506350946109 51.25) (stroke (width .05) (type default)) (layer "Edge.Cuts"))
 (gr_line (start 63.66506350946109 51.25) (end 63.80969883127822 50.956708580912725) (stroke (width .05) (type default)) (layer "Edge.Cuts"))
 (gr_line (start 63.80969883127822 50.956708580912725) (end 63.91481456572267 50.6470476127563) (stroke (width .05) (type default))
  (layer "Edge.Cuts"))
 (gr_line (start 63.91481456572267 50.6470476127563) (end 63.978612153434526 50.32631548055013) (stroke (width .05) (type default))
  (layer "Edge.Cuts"))
 (gr_line (start 63.978612153434526 50.32631548055013) (end 64.0 50.0) (stroke (width .05) (type default)) (layer "Edge.Cuts"))
 (gr_line (start 64.0 50.0) (end 63.978612153434526 49.67368451944987) (stroke (width .05) (type default)) (layer "Edge.Cuts"))
 (gr_line (start 63.978612153434526 49.67368451944987) (end 63.91481456572267 49.3529523872437) (stroke (width .05) (type default))
  (layer "Edge.Cuts"))
 (gr_line (start 63.91481456572267 49.3529523872437) (end 63.80969883127822 49.043291419087275) (stroke (width .05) (type default))
  (layer "Edge.Cuts"))
 (gr_line (start 63.80969883127822 49.043291419087275) (end 63.6650635094611 48.75) (stroke (width .05) (type default)) (layer "Edge.Cuts"))
 (gr_line (start 63.6650635094611 48.75) (end 63.48338335072809 48.4780964274782) (stroke (width .05) (type default)) (layer "Edge.Cuts"))
 (gr_line (start 63.48338335072809 48.4780964274782) (end 63.26776695296637 48.23223304703363) (stroke (width .05) (type default))
  (layer "Edge.Cuts"))
 (gr_line (start 63.26776695296637 48.23223304703363) (end 63.0219035725218 48.01661664927191) (stroke (width .05) (type default))
  (layer "Edge.Cuts"))
 (gr_line (start 63.0219035725218 48.01661664927191) (end 62.8 47.86834542243487) (stroke (width .05) (type default)) (layer "Edge.Cuts"))
 (gr_line (start 62.8 47.86834542243487) (end 62.8 46.7) (stroke (width .05) (type default)) (layer "Edge.Cuts"))
 (gr_line (start 62.8 46.7) (end 62.78887831978595 46.53031595011393) (stroke (width .05) (type default)) (layer "Edge.Cuts"))
 (gr_line (start 62.78887831978595 46.53031595011393) (end 62.75570357417579 46.363535241366726) (stroke (width .05) (type default))
  (layer "Edge.Cuts"))
 (gr_line (start 62.75570357417579 46.363535241366726) (end 62.70104339226467 46.20251153792538) (stroke (width .05) (type default))
  (layer "Edge.Cuts"))
 (gr_line (start 62.70104339226467 46.20251153792538) (end 62.62583302491977 46.05) (stroke (width .05) (type default)) (layer "Edge.Cuts"))
 (gr_line (start 62.62583302491977 46.05) (end 62.53135934237861 45.908610142288666) (stroke (width .05) (type default)) (layer "Edge.Cuts"))
 (gr_line (start 62.53135934237861 45.908610142288666) (end 62.41923881554251 45.78076118445749) (stroke (width .05) (type default))
  (layer "Edge.Cuts"))
 (gr_line (start 62.41923881554251 45.78076118445749) (end 62.29138985771134 45.668640657621395) (stroke (width .05) (type default))
  (layer "Edge.Cuts"))
 (gr_line (start 62.29138985771134 45.668640657621395) (end 62.15 45.57416697508023) (stroke (width .05) (type default)) (layer "Edge.Cuts"))
 (gr_line (start 62.15 45.57416697508023) (end 61.997488462074614 45.49895660773533) (stroke (width .05) (type default)) (layer "Edge.Cuts"))
 (gr_line (start 61.997488462074614 45.49895660773533) (end 61.83646475863328 45.44429642582421) (stroke (width .05) (type default))
  (layer "Edge.Cuts"))
 (gr_line (start 61.83646475863328 45.44429642582421) (end 61.669684049886065 45.411121680214045) (stroke (width .05) (type default))
  (layer "Edge.Cuts"))
 (gr_line (start 61.669684049886065 45.411121680214045) (end 61.66757283322946 45.410983303763615) (stroke (width .05) (type default))
  (layer "Edge.Cuts"))
 (gr_line (start 61.66757283322946 45.410983303763615) (end 61.57687846171137 44.9756503204768) (stroke (width .05) (type default))
  (layer "Edge.Cuts"))
 (gr_line (start 61.57687846171137 44.9756503204768) (end 61.5363181856797 44.831157732859225) (stroke (width .05) (type default))
  (layer "Edge.Cuts")))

